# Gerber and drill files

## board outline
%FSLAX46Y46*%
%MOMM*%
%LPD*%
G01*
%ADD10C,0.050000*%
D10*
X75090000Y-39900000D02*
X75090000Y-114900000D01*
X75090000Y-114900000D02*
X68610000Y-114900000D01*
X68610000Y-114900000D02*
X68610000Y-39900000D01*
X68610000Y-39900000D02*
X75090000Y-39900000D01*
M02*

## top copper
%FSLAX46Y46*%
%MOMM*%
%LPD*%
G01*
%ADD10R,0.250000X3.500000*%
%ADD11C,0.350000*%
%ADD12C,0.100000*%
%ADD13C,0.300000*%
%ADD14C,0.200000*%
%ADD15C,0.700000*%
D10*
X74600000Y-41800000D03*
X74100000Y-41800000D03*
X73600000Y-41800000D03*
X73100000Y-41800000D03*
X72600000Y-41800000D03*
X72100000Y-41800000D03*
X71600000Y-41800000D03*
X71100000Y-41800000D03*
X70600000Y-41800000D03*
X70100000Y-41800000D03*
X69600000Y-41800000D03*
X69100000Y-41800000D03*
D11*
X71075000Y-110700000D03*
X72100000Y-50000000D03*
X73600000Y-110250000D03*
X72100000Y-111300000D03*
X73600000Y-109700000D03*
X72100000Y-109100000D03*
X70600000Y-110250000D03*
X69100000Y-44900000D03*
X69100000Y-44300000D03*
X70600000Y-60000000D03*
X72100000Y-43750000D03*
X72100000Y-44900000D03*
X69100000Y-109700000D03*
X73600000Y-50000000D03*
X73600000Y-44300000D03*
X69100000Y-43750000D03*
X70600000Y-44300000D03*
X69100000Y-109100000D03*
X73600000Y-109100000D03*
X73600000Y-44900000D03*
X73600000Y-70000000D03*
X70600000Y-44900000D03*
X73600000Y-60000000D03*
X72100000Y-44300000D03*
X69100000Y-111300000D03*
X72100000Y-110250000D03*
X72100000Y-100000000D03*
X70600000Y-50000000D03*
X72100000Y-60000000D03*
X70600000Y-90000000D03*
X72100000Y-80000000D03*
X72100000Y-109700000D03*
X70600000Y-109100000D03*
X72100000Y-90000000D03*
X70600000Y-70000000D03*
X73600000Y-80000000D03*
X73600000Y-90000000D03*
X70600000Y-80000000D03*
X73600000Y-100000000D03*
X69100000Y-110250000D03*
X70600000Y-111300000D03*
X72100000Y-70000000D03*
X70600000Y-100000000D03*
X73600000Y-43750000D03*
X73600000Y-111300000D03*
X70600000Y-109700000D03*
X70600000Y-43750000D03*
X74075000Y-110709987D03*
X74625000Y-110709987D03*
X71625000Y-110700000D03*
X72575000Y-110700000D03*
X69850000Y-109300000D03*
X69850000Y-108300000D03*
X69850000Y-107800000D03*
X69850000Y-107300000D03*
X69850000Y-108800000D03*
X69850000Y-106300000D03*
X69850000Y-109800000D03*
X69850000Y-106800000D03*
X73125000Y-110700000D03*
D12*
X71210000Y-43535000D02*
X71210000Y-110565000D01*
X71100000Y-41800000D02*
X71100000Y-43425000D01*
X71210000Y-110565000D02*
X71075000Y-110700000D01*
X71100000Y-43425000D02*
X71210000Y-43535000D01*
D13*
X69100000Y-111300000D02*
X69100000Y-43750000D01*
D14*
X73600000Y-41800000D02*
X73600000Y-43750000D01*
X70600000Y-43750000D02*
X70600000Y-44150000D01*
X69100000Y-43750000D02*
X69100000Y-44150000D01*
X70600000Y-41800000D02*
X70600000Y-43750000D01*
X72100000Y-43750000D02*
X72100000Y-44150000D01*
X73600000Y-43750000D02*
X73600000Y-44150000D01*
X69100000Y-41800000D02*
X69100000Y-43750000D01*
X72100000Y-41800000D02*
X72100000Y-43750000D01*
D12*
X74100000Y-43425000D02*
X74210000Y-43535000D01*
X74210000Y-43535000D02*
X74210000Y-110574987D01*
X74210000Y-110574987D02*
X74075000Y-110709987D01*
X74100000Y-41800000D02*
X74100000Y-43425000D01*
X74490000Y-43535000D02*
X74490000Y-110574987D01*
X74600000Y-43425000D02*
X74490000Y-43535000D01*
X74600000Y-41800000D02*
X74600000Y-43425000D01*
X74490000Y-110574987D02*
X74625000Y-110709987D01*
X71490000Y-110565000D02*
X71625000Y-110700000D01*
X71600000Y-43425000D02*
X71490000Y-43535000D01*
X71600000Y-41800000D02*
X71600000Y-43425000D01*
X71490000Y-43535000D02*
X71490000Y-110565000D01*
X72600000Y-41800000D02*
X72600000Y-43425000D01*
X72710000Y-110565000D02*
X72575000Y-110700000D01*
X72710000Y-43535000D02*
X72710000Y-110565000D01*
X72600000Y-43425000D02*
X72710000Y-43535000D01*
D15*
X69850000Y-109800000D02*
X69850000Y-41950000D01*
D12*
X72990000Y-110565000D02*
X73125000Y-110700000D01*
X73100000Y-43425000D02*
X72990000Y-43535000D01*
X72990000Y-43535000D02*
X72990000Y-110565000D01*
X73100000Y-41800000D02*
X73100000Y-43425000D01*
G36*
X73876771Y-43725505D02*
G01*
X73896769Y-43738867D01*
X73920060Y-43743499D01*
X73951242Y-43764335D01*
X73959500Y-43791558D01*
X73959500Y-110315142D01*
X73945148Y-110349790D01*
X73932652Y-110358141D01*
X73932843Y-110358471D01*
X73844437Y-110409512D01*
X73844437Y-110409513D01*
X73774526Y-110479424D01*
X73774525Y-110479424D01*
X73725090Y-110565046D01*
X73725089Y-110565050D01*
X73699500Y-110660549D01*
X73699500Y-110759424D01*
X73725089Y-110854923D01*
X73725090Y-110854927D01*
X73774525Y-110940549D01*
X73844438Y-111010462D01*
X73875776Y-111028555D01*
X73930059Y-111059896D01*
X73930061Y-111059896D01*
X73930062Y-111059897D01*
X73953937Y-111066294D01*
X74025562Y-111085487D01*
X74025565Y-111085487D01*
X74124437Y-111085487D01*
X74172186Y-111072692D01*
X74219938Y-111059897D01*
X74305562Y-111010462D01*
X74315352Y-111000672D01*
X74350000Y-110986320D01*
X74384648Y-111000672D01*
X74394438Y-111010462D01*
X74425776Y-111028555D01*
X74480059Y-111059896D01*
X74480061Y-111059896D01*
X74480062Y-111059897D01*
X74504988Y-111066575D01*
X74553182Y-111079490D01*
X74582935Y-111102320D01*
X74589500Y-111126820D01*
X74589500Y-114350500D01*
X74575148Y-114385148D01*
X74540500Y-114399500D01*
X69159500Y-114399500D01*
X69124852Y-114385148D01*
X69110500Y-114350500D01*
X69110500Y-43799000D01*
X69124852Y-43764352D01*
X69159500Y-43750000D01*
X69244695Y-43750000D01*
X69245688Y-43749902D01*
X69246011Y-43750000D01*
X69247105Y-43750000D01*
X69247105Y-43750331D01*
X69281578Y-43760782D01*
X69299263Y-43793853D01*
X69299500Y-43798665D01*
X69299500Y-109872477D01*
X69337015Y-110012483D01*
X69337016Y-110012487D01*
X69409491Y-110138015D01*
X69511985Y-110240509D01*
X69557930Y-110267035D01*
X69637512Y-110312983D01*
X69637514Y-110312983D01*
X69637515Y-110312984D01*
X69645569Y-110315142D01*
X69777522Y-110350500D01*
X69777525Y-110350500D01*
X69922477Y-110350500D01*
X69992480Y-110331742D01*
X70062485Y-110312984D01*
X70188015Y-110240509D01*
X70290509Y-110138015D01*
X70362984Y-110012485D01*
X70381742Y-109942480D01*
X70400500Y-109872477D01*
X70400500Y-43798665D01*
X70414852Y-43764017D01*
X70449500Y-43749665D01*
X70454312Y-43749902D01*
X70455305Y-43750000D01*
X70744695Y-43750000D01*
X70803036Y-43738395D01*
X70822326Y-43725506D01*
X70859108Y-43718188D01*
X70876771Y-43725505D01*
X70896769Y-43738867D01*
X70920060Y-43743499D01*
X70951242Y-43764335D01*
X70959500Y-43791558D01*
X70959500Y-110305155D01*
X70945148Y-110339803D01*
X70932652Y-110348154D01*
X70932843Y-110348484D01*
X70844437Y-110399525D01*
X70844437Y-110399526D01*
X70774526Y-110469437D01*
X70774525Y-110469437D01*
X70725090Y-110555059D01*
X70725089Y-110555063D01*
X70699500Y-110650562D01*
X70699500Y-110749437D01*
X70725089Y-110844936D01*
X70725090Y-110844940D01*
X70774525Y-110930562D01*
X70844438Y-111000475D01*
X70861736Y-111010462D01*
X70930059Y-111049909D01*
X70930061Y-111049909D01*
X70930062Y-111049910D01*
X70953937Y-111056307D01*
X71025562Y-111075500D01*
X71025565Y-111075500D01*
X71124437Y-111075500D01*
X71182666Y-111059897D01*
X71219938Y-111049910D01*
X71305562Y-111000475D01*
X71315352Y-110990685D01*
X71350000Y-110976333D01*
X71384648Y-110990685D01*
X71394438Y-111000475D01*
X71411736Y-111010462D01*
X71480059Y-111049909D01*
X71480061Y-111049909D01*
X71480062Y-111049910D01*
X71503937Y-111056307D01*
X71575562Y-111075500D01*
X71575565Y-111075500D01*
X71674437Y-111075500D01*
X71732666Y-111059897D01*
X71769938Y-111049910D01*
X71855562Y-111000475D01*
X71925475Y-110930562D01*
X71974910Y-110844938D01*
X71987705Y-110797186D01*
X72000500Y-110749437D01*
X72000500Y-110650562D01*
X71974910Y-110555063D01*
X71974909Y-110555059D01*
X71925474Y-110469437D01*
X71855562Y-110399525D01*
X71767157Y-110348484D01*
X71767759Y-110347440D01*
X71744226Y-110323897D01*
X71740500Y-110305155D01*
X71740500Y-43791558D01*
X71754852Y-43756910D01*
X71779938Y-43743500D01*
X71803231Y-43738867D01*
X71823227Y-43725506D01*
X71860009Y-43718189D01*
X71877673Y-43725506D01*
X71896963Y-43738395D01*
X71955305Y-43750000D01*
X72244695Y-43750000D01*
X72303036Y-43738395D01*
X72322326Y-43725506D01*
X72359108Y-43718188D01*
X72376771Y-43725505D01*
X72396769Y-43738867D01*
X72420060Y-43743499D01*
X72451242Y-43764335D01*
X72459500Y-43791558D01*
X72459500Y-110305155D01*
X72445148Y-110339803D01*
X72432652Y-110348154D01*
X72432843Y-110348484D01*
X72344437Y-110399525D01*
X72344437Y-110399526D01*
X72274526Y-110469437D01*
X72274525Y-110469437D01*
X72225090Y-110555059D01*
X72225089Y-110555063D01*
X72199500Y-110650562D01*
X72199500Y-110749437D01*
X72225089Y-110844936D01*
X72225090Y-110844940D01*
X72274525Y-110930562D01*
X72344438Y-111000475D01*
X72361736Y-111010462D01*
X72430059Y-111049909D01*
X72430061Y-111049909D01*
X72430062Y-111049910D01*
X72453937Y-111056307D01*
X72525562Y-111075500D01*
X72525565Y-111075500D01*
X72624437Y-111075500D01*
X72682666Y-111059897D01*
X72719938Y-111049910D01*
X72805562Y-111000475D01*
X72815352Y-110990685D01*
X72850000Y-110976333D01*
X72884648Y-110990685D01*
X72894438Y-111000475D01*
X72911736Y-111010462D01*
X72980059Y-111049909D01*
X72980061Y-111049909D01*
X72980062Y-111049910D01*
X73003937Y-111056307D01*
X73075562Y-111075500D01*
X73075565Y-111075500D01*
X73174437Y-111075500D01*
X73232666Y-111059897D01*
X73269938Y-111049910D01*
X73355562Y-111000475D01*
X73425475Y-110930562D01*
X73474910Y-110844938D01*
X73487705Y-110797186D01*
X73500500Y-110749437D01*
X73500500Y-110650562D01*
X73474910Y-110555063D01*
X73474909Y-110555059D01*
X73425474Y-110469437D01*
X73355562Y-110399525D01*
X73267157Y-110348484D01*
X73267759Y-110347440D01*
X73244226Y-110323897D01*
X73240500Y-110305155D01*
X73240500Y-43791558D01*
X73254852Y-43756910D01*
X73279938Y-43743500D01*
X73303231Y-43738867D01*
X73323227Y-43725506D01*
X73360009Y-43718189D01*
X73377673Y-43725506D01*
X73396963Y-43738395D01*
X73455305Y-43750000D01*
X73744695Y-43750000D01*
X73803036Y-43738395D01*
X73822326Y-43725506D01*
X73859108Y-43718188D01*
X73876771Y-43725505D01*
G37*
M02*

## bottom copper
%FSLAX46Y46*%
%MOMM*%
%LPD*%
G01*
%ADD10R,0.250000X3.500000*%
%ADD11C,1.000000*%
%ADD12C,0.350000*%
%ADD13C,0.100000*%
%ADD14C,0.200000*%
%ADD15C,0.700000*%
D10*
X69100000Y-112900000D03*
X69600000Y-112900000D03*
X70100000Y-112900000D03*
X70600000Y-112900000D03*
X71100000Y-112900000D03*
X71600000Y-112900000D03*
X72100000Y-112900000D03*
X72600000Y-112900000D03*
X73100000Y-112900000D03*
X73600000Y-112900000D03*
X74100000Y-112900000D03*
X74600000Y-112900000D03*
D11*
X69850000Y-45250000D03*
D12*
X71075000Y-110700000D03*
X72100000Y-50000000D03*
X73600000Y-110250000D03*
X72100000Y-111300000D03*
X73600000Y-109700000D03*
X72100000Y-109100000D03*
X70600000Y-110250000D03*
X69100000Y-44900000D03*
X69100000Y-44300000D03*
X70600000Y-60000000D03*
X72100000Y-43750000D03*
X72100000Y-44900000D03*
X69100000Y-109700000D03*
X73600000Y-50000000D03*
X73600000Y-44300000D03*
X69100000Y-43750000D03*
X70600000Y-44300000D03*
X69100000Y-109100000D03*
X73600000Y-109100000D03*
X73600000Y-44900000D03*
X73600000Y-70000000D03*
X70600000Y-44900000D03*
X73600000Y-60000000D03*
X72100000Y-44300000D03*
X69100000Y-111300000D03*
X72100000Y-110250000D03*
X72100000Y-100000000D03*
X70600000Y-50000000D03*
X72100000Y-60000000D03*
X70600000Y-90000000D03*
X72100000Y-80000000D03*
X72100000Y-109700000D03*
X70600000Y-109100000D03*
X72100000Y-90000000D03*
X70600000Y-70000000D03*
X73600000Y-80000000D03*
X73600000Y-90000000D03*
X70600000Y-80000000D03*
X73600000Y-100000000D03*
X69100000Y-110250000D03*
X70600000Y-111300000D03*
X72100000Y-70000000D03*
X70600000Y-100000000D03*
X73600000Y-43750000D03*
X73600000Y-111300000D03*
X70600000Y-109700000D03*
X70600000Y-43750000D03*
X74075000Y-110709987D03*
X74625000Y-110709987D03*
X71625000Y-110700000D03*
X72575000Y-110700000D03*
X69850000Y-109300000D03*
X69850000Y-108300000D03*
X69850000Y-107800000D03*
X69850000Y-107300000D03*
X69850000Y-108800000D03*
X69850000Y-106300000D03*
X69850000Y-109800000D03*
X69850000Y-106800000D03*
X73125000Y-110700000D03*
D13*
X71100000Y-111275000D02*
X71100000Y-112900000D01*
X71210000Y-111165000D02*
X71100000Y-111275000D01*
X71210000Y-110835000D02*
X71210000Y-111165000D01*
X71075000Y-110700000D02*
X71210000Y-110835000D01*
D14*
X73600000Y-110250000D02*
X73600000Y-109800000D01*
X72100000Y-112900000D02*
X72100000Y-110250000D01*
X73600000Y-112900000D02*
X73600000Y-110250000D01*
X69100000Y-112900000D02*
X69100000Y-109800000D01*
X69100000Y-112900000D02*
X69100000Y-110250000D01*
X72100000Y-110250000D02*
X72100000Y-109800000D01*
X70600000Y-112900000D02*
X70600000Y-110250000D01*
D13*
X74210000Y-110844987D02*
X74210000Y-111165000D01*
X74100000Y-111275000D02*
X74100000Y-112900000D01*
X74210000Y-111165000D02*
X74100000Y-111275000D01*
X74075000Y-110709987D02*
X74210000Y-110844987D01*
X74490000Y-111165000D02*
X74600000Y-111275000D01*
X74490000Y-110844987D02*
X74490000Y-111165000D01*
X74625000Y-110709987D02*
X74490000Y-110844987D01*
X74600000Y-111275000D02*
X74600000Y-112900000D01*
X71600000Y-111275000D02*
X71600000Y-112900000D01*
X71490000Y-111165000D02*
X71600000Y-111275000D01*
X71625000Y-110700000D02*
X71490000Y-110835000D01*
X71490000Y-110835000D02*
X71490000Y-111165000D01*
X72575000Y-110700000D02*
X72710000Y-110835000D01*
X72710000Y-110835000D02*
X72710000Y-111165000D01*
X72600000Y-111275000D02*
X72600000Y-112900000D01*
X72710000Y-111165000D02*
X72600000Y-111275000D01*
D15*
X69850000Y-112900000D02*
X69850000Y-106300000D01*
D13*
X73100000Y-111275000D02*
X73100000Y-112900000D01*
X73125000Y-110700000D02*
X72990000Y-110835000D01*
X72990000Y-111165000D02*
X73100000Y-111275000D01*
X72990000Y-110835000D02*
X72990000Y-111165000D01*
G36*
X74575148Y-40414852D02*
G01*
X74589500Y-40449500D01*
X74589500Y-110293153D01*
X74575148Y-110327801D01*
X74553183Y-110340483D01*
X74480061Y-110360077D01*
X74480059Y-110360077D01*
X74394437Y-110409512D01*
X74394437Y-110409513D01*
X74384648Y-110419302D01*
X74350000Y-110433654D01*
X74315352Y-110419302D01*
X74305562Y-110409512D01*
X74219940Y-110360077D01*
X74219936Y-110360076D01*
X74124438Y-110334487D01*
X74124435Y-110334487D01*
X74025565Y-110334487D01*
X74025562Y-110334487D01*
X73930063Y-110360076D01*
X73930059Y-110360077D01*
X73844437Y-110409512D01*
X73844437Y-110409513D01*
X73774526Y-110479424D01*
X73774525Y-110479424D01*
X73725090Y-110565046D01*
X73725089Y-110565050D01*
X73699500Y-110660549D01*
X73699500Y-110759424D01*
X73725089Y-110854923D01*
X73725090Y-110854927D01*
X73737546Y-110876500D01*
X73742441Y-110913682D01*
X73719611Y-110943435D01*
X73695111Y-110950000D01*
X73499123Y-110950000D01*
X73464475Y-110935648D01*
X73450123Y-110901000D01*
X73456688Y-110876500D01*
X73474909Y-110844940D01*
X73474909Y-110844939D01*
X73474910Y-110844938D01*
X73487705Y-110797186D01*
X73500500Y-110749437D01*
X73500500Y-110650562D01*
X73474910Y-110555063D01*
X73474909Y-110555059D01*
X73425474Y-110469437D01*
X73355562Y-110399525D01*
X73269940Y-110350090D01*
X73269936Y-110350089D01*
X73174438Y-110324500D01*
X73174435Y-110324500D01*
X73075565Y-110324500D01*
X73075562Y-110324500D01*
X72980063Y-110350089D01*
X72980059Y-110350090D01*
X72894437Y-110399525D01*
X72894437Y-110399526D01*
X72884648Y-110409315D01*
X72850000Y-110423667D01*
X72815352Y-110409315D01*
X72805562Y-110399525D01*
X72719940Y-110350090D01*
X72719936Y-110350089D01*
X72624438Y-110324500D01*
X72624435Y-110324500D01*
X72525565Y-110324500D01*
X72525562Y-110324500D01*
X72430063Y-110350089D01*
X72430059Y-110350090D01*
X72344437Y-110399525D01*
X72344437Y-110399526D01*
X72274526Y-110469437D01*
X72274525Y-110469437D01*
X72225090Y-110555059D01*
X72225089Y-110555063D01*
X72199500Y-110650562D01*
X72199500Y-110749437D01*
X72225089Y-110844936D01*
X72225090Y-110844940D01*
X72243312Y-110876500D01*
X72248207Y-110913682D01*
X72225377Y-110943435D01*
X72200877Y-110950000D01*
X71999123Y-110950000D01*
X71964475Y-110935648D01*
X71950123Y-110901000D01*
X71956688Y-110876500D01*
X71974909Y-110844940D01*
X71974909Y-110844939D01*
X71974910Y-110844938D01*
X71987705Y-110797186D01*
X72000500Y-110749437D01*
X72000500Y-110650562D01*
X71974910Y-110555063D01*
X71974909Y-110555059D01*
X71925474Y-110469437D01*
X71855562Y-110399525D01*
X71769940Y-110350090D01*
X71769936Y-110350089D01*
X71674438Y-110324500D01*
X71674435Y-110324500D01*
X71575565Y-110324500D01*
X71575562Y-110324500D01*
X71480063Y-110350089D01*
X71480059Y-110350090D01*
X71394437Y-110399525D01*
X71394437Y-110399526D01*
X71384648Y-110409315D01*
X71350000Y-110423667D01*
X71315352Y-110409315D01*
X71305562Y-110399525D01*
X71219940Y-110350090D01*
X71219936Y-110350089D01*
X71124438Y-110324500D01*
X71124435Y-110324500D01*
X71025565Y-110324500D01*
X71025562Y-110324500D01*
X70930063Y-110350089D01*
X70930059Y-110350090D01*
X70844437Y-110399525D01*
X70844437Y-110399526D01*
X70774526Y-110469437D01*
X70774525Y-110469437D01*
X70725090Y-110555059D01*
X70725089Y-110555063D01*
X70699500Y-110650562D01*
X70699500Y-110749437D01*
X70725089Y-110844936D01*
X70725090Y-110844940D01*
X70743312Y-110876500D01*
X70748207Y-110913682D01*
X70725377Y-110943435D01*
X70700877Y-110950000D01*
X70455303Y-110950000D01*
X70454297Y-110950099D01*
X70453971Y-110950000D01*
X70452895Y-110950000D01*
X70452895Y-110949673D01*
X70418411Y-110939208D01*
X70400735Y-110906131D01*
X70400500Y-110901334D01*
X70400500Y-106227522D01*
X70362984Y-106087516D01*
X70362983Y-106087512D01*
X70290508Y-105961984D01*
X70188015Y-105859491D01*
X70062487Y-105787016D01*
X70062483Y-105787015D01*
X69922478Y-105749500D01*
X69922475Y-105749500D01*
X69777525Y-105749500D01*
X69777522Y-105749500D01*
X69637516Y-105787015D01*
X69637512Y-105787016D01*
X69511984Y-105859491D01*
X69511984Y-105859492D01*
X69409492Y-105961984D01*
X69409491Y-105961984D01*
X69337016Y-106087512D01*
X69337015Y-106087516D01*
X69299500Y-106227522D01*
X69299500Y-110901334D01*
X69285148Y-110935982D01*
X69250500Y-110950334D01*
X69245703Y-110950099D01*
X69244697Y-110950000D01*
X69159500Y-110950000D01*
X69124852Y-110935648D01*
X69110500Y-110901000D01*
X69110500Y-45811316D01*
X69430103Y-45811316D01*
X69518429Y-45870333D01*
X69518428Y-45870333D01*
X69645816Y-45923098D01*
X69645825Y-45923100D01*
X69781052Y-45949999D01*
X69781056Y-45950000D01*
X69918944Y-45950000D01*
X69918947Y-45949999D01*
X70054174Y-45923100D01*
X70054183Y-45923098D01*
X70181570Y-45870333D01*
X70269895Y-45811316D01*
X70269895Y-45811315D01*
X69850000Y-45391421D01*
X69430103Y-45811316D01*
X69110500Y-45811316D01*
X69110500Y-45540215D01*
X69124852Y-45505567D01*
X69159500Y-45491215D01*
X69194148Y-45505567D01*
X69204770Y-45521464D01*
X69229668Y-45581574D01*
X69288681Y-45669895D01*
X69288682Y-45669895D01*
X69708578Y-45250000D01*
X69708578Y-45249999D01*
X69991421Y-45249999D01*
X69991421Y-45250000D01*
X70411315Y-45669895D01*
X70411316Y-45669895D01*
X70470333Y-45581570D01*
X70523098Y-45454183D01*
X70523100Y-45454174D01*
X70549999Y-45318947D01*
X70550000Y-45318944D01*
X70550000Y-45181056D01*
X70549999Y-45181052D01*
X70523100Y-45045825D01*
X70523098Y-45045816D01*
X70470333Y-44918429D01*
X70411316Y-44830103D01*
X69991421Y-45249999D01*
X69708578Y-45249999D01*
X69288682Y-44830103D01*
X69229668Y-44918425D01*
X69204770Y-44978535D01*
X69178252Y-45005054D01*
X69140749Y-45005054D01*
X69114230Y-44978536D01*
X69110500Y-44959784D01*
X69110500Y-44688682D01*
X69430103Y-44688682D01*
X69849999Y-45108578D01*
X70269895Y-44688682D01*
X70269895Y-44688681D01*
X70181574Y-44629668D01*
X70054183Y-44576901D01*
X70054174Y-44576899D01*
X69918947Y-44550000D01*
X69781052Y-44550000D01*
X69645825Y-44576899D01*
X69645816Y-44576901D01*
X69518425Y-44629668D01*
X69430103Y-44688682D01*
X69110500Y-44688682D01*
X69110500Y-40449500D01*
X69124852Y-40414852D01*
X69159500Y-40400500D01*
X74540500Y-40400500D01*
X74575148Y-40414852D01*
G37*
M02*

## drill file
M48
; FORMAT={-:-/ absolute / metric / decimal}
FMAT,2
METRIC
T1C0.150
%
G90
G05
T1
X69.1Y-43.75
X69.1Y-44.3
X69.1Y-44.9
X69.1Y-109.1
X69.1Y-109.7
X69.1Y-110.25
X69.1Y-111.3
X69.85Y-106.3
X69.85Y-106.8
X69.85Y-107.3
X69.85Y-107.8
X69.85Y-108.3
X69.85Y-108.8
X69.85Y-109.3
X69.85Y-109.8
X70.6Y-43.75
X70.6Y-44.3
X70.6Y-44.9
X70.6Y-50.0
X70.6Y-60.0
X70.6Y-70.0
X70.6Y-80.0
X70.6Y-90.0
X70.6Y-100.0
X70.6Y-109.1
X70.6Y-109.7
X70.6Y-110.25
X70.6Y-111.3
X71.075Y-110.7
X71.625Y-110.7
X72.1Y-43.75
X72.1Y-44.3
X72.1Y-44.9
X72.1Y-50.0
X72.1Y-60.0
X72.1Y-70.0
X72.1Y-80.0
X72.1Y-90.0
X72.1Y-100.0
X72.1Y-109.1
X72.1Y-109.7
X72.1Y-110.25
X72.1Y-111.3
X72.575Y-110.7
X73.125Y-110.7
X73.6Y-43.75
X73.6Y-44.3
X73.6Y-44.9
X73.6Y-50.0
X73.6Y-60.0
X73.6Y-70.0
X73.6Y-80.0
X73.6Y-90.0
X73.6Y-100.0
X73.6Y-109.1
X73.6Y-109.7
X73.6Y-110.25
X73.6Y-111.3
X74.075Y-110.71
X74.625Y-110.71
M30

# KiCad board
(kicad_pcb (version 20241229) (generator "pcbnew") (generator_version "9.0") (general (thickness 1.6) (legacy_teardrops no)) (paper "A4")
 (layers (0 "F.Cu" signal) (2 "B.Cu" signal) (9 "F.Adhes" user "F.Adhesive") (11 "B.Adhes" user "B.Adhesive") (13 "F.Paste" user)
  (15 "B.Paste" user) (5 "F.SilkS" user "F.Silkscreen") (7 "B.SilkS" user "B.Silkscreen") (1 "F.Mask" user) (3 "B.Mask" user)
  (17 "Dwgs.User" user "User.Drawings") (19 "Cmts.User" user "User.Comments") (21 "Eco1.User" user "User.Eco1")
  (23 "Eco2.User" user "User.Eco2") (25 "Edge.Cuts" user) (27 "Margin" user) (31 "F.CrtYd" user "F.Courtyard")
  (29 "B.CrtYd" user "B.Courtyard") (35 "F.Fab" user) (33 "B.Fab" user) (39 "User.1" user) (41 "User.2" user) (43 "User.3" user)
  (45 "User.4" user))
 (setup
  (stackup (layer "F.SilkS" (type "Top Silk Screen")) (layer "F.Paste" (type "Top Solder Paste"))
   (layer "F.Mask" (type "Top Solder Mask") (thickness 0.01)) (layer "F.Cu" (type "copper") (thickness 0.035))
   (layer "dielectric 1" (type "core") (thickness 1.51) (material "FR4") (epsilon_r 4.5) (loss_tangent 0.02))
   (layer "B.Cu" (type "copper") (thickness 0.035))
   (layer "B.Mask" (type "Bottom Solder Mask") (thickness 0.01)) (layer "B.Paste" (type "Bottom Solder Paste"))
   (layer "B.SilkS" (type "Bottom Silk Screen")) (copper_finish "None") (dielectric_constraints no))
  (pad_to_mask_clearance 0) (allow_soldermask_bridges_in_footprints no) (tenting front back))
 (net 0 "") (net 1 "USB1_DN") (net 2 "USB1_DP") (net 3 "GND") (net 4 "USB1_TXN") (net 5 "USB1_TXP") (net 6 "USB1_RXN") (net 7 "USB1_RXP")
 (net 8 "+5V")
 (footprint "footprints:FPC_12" (layer "F.Cu") (at 71.85 41.8)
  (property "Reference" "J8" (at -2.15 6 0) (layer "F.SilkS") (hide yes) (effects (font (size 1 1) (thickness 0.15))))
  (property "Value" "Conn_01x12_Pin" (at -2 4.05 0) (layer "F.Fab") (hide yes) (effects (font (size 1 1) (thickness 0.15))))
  (pad "1" smd rect (at 2.75 0) (size 0.25 3.5) (layers "F.Cu" "F.Mask" "F.Paste") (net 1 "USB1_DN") (thermal_bridge_angle 45))
  (pad "2" smd rect (at 2.25 0) (size 0.25 3.5) (layers "F.Cu" "F.Mask" "F.Paste") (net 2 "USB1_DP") (thermal_bridge_angle 45))
  (pad "3" smd rect (at 1.75 0) (size 0.25 3.5) (layers "F.Cu" "F.Mask" "F.Paste") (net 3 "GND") (thermal_bridge_angle 45))
  (pad "4" smd rect (at 1.25 0) (size 0.25 3.5) (layers "F.Cu" "F.Mask" "F.Paste") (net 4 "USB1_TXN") (thermal_bridge_angle 45))
  (pad "5" smd rect (at 0.75 0) (size 0.25 3.5) (layers "F.Cu" "F.Mask" "F.Paste") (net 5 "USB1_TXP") (thermal_bridge_angle 45))
  (pad "6" smd rect (at 0.25 0) (size 0.25 3.5) (layers "F.Cu" "F.Mask" "F.Paste") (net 3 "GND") (thermal_bridge_angle 45))
  (pad "7" smd rect (at -0.25 0) (size 0.25 3.5) (layers "F.Cu" "F.Mask" "F.Paste") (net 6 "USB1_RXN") (thermal_bridge_angle 45))
  (pad "8" smd rect (at -0.75 0) (size 0.25 3.5) (layers "F.Cu" "F.Mask" "F.Paste") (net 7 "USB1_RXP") (thermal_bridge_angle 45))
  (pad "9" smd rect (at -1.25 0) (size 0.25 3.5) (layers "F.Cu" "F.Mask" "F.Paste") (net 3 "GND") (thermal_bridge_angle 45))
  (pad "10" smd rect (at -1.75 0) (size 0.25 3.5) (layers "F.Cu" "F.Mask" "F.Paste") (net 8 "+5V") (thermal_bridge_angle 45))
  (pad "11" smd rect (at -2.25 0) (size 0.25 3.5) (layers "F.Cu" "F.Mask" "F.Paste") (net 8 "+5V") (thermal_bridge_angle 45))
  (pad "12" smd rect (at -2.75 0) (size 0.25 3.5) (layers "F.Cu" "F.Mask" "F.Paste") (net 3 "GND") (thermal_bridge_angle 45)))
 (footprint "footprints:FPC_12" (layer "B.Cu") (at 71.85 112.9 180)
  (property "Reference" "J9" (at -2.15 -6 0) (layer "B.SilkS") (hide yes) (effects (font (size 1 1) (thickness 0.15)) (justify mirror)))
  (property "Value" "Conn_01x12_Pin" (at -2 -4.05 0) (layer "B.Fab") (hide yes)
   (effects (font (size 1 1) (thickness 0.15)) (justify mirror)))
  (pad "1" smd rect (at 2.75 0 180) (size 0.25 3.5) (layers "B.Cu" "B.Mask" "B.Paste") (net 3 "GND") (thermal_bridge_angle 45))
  (pad "2" smd rect (at 2.25 0 180) (size 0.25 3.5) (layers "B.Cu" "B.Mask" "B.Paste") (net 8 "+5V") (thermal_bridge_angle 45))
  (pad "3" smd rect (at 1.75 0 180) (size 0.25 3.5) (layers "B.Cu" "B.Mask" "B.Paste") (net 8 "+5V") (thermal_bridge_angle 45))
  (pad "4" smd rect (at 1.25 0 180) (size 0.25 3.5) (layers "B.Cu" "B.Mask" "B.Paste") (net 3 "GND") (thermal_bridge_angle 45))
  (pad "5" smd rect (at 0.75 0 180) (size 0.25 3.5) (layers "B.Cu" "B.Mask" "B.Paste") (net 7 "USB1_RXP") (thermal_bridge_angle 45))
  (pad "6" smd rect (at 0.25 0 180) (size 0.25 3.5) (layers "B.Cu" "B.Mask" "B.Paste") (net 6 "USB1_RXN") (thermal_bridge_angle 45))
  (pad "7" smd rect (at -0.25 0 180) (size 0.25 3.5) (layers "B.Cu" "B.Mask" "B.Paste") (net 3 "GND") (thermal_bridge_angle 45))
  (pad "8" smd rect (at -0.75 0 180) (size 0.25 3.5) (layers "B.Cu" "B.Mask" "B.Paste") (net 5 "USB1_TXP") (thermal_bridge_angle 45))
  (pad "9" smd rect (at -1.25 0 180) (size 0.25 3.5) (layers "B.Cu" "B.Mask" "B.Paste") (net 4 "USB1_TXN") (thermal_bridge_angle 45))
  (pad "10" smd rect (at -1.75 0 180) (size 0.25 3.5) (layers "B.Cu" "B.Mask" "B.Paste") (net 3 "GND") (thermal_bridge_angle 45))
  (pad "11" smd rect (at -2.25 0 180) (size 0.25 3.5) (layers "B.Cu" "B.Mask" "B.Paste") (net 2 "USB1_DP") (thermal_bridge_angle 45))
  (pad "12" smd rect (at -2.75 0 180) (size 0.25 3.5) (layers "B.Cu" "B.Mask" "B.Paste") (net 1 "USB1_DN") (thermal_bridge_angle 45)))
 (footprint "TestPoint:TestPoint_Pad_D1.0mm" (layer "B.Cu") (at 69.85 45.25 180)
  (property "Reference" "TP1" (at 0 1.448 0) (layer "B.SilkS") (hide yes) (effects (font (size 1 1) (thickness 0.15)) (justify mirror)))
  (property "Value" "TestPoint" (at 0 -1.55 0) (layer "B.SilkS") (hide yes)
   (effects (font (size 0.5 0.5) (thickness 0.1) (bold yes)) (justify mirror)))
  (pad "1" smd circle (at 0 0 180) (size 1 1) (layers "B.Cu" "B.Mask") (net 3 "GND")))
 (gr_line (start 75.09 39.9) (end 75.09 114.9) (stroke (width 0.05) (type solid)) (layer "Edge.Cuts"))
 (gr_line (start 75.09 114.9) (end 68.61 114.9) (stroke (width 0.05) (type solid)) (layer "Edge.Cuts"))
 (gr_line (start 68.61 114.9) (end 68.61 39.9) (stroke (width 0.05) (type solid)) (layer "Edge.Cuts"))
 (gr_line (start 68.61 39.9) (end 75.09 39.9) (stroke (width 0.05) (type solid)) (layer "Edge.Cuts"))
 (segment (start 71.21 43.535) (end 71.21 110.565) (width 0.1) (layer "F.Cu") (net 7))
 (segment (start 71.1 41.8) (end 71.1 43.425) (width 0.1) (layer "F.Cu") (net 7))
 (segment (start 71.21 110.565) (end 71.075 110.7) (width 0.1) (layer "F.Cu") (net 7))
 (segment (start 71.1 43.425) (end 71.21 43.535) (width 0.1) (layer "F.Cu") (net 7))
 (via (at 71.075 110.7) (size 0.35) (drill 0.15) (layers "F.Cu" "B.Cu") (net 7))
 (segment (start 71.1 111.275) (end 71.1 112.9) (width 0.1) (layer "B.Cu") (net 7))
 (segment (start 71.21 111.165) (end 71.1 111.275) (width 0.1) (layer "B.Cu") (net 7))
 (segment (start 71.21 110.835) (end 71.21 111.165) (width 0.1) (layer "B.Cu") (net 7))
 (segment (start 71.075 110.7) (end 71.21 110.835) (width 0.1) (layer "B.Cu") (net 7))
 (segment (start 69.1 111.3) (end 69.1 43.75) (width 0.3) (layer "F.Cu") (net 3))
 (segment (start 73.6 41.8) (end 73.6 43.75) (width 0.2) (layer "F.Cu") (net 3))
 (segment (start 70.6 43.75) (end 70.6 44.15) (width 0.2) (layer "F.Cu") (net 3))
 (segment (start 69.1 43.75) (end 69.1 44.15) (width 0.2) (layer "F.Cu") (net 3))
 (segment (start 70.6 41.8) (end 70.6 43.75) (width 0.2) (layer "F.Cu") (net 3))
 (segment (start 72.1 43.75) (end 72.1 44.15) (width 0.2) (layer "F.Cu") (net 3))
 (segment (start 73.6 43.75) (end 73.6 44.15) (width 0.2) (layer "F.Cu") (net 3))
 (segment (start 69.1 41.8) (end 69.1 43.75) (width 0.2) (layer "F.Cu") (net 3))
 (segment (start 72.1 41.8) (end 72.1 43.75) (width 0.2) (layer "F.Cu") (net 3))
 (via (at 72.1 50) (size 0.35) (drill 0.15) (layers "F.Cu" "B.Cu") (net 3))
 (via (at 73.6 110.25) (size 0.35) (drill 0.15) (layers "F.Cu" "B.Cu") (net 3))
 (via (at 72.1 111.3) (size 0.35) (drill 0.15) (layers "F.Cu" "B.Cu") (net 3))
 (via (at 73.6 109.7) (size 0.35) (drill 0.15) (layers "F.Cu" "B.Cu") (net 3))
 (via (at 72.1 109.1) (size 0.35) (drill 0.15) (layers "F.Cu" "B.Cu") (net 3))
 (via (at 70.6 110.25) (size 0.35) (drill 0.15) (layers "F.Cu" "B.Cu") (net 3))
 (via (at 69.1 44.9) (size 0.35) (drill 0.15) (layers "F.Cu" "B.Cu") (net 3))
 (via (at 69.1 44.3) (size 0.35) (drill 0.15) (layers "F.Cu" "B.Cu") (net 3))
 (via (at 70.6 60) (size 0.35) (drill 0.15) (layers "F.Cu" "B.Cu") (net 3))
 (via (at 72.1 43.75) (size 0.35) (drill 0.15) (layers "F.Cu" "B.Cu") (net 3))
 (via (at 72.1 44.9) (size 0.35) (drill 0.15) (layers "F.Cu" "B.Cu") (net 3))
 (via (at 69.1 109.7) (size 0.35) (drill 0.15) (layers "F.Cu" "B.Cu") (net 3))
 (via (at 73.6 50) (size 0.35) (drill 0.15) (layers "F.Cu" "B.Cu") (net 3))
 (via (at 73.6 44.3) (size 0.35) (drill 0.15) (layers "F.Cu" "B.Cu") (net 3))
 (via (at 69.1 43.75) (size 0.35) (drill 0.15) (layers "F.Cu" "B.Cu") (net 3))
 (via (at 70.6 44.3) (size 0.35) (drill 0.15) (layers "F.Cu" "B.Cu") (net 3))
 (via (at 69.1 109.1) (size 0.35) (drill 0.15) (layers "F.Cu" "B.Cu") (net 3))
 (via (at 73.6 109.1) (size 0.35) (drill 0.15) (layers "F.Cu" "B.Cu") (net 3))
 (via (at 73.6 44.9) (size 0.35) (drill 0.15) (layers "F.Cu" "B.Cu") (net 3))
 (via (at 73.6 70) (size 0.35) (drill 0.15) (layers "F.Cu" "B.Cu") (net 3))
 (via (at 70.6 44.9) (size 0.35) (drill 0.15) (layers "F.Cu" "B.Cu") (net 3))
 (via (at 73.6 60) (size 0.35) (drill 0.15) (layers "F.Cu" "B.Cu") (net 3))
 (via (at 72.1 44.3) (size 0.35) (drill 0.15) (layers "F.Cu" "B.Cu") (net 3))
 (via (at 69.1 111.3) (size 0.35) (drill 0.15) (layers "F.Cu" "B.Cu") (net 3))
 (via (at 72.1 110.25) (size 0.35) (drill 0.15) (layers "F.Cu" "B.Cu") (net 3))
 (via (at 72.1 100) (size 0.35) (drill 0.15) (layers "F.Cu" "B.Cu") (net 3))
 (via (at 70.6 50) (size 0.35) (drill 0.15) (layers "F.Cu" "B.Cu") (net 3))
 (via (at 72.1 60) (size 0.35) (drill 0.15) (layers "F.Cu" "B.Cu") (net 3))
 (via (at 70.6 90) (size 0.35) (drill 0.15) (layers "F.Cu" "B.Cu") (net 3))
 (via (at 72.1 80) (size 0.35) (drill 0.15) (layers "F.Cu" "B.Cu") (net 3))
 (via (at 72.1 109.7) (size 0.35) (drill 0.15) (layers "F.Cu" "B.Cu") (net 3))
 (via (at 70.6 109.1) (size 0.35) (drill 0.15) (layers "F.Cu" "B.Cu") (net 3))
 (via (at 72.1 90) (size 0.35) (drill 0.15) (layers "F.Cu" "B.Cu") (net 3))
 (via (at 70.6 70) (size 0.35) (drill 0.15) (layers "F.Cu" "B.Cu") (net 3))
 (via (at 73.6 80) (size 0.35) (drill 0.15) (layers "F.Cu" "B.Cu") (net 3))
 (via (at 73.6 90) (size 0.35) (drill 0.15) (layers "F.Cu" "B.Cu") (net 3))
 (via (at 70.6 80) (size 0.35) (drill 0.15) (layers "F.Cu" "B.Cu") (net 3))
 (via (at 73.6 100) (size 0.35) (drill 0.15) (layers "F.Cu" "B.Cu") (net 3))
 (via (at 69.1 110.25) (size 0.35) (drill 0.15) (layers "F.Cu" "B.Cu") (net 3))
 (via (at 70.6 111.3) (size 0.35) (drill 0.15) (layers "F.Cu" "B.Cu") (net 3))
 (via (at 72.1 70) (size 0.35) (drill 0.15) (layers "F.Cu" "B.Cu") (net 3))
 (via (at 70.6 100) (size 0.35) (drill 0.15) (layers "F.Cu" "B.Cu") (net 3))
 (via (at 73.6 43.75) (size 0.35) (drill 0.15) (layers "F.Cu" "B.Cu") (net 3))
 (via (at 73.6 111.3) (size 0.35) (drill 0.15) (layers "F.Cu" "B.Cu") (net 3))
 (via (at 70.6 109.7) (size 0.35) (drill 0.15) (layers "F.Cu" "B.Cu") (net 3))
 (via (at 70.6 43.75) (size 0.35) (drill 0.15) (layers "F.Cu" "B.Cu") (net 3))
 (segment (start 73.6 110.25) (end 73.6 109.8) (width 0.2) (layer "B.Cu") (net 3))
 (segment (start 72.1 112.9) (end 72.1 110.25) (width 0.2) (layer "B.Cu") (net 3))
 (segment (start 73.6 112.9) (end 73.6 110.25) (width 0.2) (layer "B.Cu") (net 3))
 (segment (start 69.1 112.9) (end 69.1 109.8) (width 0.2) (layer "B.Cu") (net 3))
 (segment (start 69.1 112.9) (end 69.1 110.25) (width 0.2) (layer "B.Cu") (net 3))
 (segment (start 72.1 110.25) (end 72.1 109.8) (width 0.2) (layer "B.Cu") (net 3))
 (segment (start 70.6 112.9) (end 70.6 110.25) (width 0.2) (layer "B.Cu") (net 3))
 (segment (start 74.1 43.425) (end 74.21 43.535) (width 0.1) (layer "F.Cu") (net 2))
 (segment (start 74.21 43.535) (end 74.21 110.574987) (width 0.1) (layer "F.Cu") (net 2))
 (segment (start 74.21 110.574987) (end 74.075 110.709987) (width 0.1) (layer "F.Cu") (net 2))
 (segment (start 74.1 41.8) (end 74.1 43.425) (width 0.1) (layer "F.Cu") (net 2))
 (via (at 74.075 110.709987) (size 0.35) (drill 0.15) (layers "F.Cu" "B.Cu") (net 2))
 (segment (start 74.21 110.844987) (end 74.21 111.165) (width 0.1) (layer "B.Cu") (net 2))
 (segment (start 74.1 111.275) (end 74.1 112.9) (width 0.1) (layer "B.Cu") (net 2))
 (segment (start 74.21 111.165) (end 74.1 111.275) (width 0.1) (layer "B.Cu") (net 2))
 (segment (start 74.075 110.709987) (end 74.21 110.844987) (width 0.1) (layer "B.Cu") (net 2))
 (segment (start 74.49 43.535) (end 74.49 110.574987) (width 0.1) (layer "F.Cu") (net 1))
 (segment (start 74.6 43.425) (end 74.49 43.535) (width 0.1) (layer "F.Cu") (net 1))
 (segment (start 74.6 41.8) (end 74.6 43.425) (width 0.1) (layer "F.Cu") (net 1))
 (segment (start 74.49 110.574987) (end 74.625 110.709987) (width 0.1) (layer "F.Cu") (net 1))
 (via (at 74.625 110.709987) (size 0.35) (drill 0.15) (layers "F.Cu" "B.Cu") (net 1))
 (segment (start 74.49 111.165) (end 74.6 111.275) (width 0.1) (layer "B.Cu") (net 1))
 (segment (start 74.49 110.844987) (end 74.49 111.165) (width 0.1) (layer "B.Cu") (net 1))
 (segment (start 74.625 110.709987) (end 74.49 110.844987) (width 0.1) (layer "B.Cu") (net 1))
 (segment (start 74.6 111.275) (end 74.6 112.9) (width 0.1) (layer "B.Cu") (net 1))
 (segment (start 71.49 110.565) (end 71.625 110.7) (width 0.1) (layer "F.Cu") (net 6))
 (segment (start 71.6 43.425) (end 71.49 43.535) (width 0.1) (layer "F.Cu") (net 6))
 (segment (start 71.6 41.8) (end 71.6 43.425) (width 0.1) (layer "F.Cu") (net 6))
 (segment (start 71.49 43.535) (end 71.49 110.565) (width 0.1) (layer "F.Cu") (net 6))
 (via (at 71.625 110.7) (size 0.35) (drill 0.15) (layers "F.Cu" "B.Cu") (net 6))
 (segment (start 71.6 111.275) (end 71.6 112.9) (width 0.1) (layer "B.Cu") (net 6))
 (segment (start 71.49 111.165) (end 71.6 111.275) (width 0.1) (layer "B.Cu") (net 6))
 (segment (start 71.625 110.7) (end 71.49 110.835) (width 0.1) (layer "B.Cu") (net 6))
 (segment (start 71.49 110.835) (end 71.49 111.165) (width 0.1) (layer "B.Cu") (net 6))
 (segment (start 72.6 41.8) (end 72.6 43.425) (width 0.1) (layer "F.Cu") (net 5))
 (segment (start 72.71 110.565) (end 72.575 110.7) (width 0.1) (layer "F.Cu") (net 5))
 (segment (start 72.71 43.535) (end 72.71 110.565) (width 0.1) (layer "F.Cu") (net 5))
 (segment (start 72.6 43.425) (end 72.71 43.535) (width 0.1) (layer "F.Cu") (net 5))
 (via (at 72.575 110.7) (size 0.35) (drill 0.15) (layers "F.Cu" "B.Cu") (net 5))
 (segment (start 72.575 110.7) (end 72.71 110.835) (width 0.1) (layer "B.Cu") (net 5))
 (segment (start 72.71 110.835) (end 72.71 111.165) (width 0.1) (layer "B.Cu") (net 5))
 (segment (start 72.6 111.275) (end 72.6 112.9) (width 0.1) (layer "B.Cu") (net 5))
 (segment (start 72.71 111.165) (end 72.6 111.275) (width 0.1) (layer "B.Cu") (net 5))
 (segment (start 69.85 109.8) (end 69.85 41.95) (width 0.7) (layer "F.Cu") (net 8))
 (via (at 69.85 109.3) (size 0.35) (drill 0.15) (layers "F.Cu" "B.Cu") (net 8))
 (via (at 69.85 108.3) (size 0.35) (drill 0.15) (layers "F.Cu" "B.Cu") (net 8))
 (via (at 69.85 107.8) (size 0.35) (drill 0.15) (layers "F.Cu" "B.Cu") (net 8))
 (via (at 69.85 107.3) (size 0.35) (drill 0.15) (layers "F.Cu" "B.Cu") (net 8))
 (via (at 69.85 108.8) (size 0.35) (drill 0.15) (layers "F.Cu" "B.Cu") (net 8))
 (via (at 69.85 106.3) (size 0.35) (drill 0.15) (layers "F.Cu" "B.Cu") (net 8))
 (via (at 69.85 109.8) (size 0.35) (drill 0.15) (layers "F.Cu" "B.Cu") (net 8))
 (via (at 69.85 106.8) (size 0.35) (drill 0.15) (layers "F.Cu" "B.Cu") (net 8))
 (segment (start 69.85 112.9) (end 69.85 106.3) (width 0.7) (layer "B.Cu") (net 8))
 (segment (start 72.99 110.565) (end 73.125 110.7) (width 0.1) (layer "F.Cu") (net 4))
 (segment (start 73.1 43.425) (end 72.99 43.535) (width 0.1) (layer "F.Cu") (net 4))
 (segment (start 72.99 43.535) (end 72.99 110.565) (width 0.1) (layer "F.Cu") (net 4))
 (segment (start 73.1 41.8) (end 73.1 43.425) (width 0.1) (layer "F.Cu") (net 4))
 (via (at 73.125 110.7) (size 0.35) (drill 0.15) (layers "F.Cu" "B.Cu") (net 4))
 (segment (start 73.1 111.275) (end 73.1 112.9) (width 0.1) (layer "B.Cu") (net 4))
 (segment (start 73.125 110.7) (end 72.99 110.835) (width 0.1) (layer "B.Cu") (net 4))
 (segment (start 72.99 111.165) (end 73.1 111.275) (width 0.1) (layer "B.Cu") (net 4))
 (segment (start 72.99 110.835) (end 72.99 111.165) (width 0.1) (layer "B.Cu") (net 4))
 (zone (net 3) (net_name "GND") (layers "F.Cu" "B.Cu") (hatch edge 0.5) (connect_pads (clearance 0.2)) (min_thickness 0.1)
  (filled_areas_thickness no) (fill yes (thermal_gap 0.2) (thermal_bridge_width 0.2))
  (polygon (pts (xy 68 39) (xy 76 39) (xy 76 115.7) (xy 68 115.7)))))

